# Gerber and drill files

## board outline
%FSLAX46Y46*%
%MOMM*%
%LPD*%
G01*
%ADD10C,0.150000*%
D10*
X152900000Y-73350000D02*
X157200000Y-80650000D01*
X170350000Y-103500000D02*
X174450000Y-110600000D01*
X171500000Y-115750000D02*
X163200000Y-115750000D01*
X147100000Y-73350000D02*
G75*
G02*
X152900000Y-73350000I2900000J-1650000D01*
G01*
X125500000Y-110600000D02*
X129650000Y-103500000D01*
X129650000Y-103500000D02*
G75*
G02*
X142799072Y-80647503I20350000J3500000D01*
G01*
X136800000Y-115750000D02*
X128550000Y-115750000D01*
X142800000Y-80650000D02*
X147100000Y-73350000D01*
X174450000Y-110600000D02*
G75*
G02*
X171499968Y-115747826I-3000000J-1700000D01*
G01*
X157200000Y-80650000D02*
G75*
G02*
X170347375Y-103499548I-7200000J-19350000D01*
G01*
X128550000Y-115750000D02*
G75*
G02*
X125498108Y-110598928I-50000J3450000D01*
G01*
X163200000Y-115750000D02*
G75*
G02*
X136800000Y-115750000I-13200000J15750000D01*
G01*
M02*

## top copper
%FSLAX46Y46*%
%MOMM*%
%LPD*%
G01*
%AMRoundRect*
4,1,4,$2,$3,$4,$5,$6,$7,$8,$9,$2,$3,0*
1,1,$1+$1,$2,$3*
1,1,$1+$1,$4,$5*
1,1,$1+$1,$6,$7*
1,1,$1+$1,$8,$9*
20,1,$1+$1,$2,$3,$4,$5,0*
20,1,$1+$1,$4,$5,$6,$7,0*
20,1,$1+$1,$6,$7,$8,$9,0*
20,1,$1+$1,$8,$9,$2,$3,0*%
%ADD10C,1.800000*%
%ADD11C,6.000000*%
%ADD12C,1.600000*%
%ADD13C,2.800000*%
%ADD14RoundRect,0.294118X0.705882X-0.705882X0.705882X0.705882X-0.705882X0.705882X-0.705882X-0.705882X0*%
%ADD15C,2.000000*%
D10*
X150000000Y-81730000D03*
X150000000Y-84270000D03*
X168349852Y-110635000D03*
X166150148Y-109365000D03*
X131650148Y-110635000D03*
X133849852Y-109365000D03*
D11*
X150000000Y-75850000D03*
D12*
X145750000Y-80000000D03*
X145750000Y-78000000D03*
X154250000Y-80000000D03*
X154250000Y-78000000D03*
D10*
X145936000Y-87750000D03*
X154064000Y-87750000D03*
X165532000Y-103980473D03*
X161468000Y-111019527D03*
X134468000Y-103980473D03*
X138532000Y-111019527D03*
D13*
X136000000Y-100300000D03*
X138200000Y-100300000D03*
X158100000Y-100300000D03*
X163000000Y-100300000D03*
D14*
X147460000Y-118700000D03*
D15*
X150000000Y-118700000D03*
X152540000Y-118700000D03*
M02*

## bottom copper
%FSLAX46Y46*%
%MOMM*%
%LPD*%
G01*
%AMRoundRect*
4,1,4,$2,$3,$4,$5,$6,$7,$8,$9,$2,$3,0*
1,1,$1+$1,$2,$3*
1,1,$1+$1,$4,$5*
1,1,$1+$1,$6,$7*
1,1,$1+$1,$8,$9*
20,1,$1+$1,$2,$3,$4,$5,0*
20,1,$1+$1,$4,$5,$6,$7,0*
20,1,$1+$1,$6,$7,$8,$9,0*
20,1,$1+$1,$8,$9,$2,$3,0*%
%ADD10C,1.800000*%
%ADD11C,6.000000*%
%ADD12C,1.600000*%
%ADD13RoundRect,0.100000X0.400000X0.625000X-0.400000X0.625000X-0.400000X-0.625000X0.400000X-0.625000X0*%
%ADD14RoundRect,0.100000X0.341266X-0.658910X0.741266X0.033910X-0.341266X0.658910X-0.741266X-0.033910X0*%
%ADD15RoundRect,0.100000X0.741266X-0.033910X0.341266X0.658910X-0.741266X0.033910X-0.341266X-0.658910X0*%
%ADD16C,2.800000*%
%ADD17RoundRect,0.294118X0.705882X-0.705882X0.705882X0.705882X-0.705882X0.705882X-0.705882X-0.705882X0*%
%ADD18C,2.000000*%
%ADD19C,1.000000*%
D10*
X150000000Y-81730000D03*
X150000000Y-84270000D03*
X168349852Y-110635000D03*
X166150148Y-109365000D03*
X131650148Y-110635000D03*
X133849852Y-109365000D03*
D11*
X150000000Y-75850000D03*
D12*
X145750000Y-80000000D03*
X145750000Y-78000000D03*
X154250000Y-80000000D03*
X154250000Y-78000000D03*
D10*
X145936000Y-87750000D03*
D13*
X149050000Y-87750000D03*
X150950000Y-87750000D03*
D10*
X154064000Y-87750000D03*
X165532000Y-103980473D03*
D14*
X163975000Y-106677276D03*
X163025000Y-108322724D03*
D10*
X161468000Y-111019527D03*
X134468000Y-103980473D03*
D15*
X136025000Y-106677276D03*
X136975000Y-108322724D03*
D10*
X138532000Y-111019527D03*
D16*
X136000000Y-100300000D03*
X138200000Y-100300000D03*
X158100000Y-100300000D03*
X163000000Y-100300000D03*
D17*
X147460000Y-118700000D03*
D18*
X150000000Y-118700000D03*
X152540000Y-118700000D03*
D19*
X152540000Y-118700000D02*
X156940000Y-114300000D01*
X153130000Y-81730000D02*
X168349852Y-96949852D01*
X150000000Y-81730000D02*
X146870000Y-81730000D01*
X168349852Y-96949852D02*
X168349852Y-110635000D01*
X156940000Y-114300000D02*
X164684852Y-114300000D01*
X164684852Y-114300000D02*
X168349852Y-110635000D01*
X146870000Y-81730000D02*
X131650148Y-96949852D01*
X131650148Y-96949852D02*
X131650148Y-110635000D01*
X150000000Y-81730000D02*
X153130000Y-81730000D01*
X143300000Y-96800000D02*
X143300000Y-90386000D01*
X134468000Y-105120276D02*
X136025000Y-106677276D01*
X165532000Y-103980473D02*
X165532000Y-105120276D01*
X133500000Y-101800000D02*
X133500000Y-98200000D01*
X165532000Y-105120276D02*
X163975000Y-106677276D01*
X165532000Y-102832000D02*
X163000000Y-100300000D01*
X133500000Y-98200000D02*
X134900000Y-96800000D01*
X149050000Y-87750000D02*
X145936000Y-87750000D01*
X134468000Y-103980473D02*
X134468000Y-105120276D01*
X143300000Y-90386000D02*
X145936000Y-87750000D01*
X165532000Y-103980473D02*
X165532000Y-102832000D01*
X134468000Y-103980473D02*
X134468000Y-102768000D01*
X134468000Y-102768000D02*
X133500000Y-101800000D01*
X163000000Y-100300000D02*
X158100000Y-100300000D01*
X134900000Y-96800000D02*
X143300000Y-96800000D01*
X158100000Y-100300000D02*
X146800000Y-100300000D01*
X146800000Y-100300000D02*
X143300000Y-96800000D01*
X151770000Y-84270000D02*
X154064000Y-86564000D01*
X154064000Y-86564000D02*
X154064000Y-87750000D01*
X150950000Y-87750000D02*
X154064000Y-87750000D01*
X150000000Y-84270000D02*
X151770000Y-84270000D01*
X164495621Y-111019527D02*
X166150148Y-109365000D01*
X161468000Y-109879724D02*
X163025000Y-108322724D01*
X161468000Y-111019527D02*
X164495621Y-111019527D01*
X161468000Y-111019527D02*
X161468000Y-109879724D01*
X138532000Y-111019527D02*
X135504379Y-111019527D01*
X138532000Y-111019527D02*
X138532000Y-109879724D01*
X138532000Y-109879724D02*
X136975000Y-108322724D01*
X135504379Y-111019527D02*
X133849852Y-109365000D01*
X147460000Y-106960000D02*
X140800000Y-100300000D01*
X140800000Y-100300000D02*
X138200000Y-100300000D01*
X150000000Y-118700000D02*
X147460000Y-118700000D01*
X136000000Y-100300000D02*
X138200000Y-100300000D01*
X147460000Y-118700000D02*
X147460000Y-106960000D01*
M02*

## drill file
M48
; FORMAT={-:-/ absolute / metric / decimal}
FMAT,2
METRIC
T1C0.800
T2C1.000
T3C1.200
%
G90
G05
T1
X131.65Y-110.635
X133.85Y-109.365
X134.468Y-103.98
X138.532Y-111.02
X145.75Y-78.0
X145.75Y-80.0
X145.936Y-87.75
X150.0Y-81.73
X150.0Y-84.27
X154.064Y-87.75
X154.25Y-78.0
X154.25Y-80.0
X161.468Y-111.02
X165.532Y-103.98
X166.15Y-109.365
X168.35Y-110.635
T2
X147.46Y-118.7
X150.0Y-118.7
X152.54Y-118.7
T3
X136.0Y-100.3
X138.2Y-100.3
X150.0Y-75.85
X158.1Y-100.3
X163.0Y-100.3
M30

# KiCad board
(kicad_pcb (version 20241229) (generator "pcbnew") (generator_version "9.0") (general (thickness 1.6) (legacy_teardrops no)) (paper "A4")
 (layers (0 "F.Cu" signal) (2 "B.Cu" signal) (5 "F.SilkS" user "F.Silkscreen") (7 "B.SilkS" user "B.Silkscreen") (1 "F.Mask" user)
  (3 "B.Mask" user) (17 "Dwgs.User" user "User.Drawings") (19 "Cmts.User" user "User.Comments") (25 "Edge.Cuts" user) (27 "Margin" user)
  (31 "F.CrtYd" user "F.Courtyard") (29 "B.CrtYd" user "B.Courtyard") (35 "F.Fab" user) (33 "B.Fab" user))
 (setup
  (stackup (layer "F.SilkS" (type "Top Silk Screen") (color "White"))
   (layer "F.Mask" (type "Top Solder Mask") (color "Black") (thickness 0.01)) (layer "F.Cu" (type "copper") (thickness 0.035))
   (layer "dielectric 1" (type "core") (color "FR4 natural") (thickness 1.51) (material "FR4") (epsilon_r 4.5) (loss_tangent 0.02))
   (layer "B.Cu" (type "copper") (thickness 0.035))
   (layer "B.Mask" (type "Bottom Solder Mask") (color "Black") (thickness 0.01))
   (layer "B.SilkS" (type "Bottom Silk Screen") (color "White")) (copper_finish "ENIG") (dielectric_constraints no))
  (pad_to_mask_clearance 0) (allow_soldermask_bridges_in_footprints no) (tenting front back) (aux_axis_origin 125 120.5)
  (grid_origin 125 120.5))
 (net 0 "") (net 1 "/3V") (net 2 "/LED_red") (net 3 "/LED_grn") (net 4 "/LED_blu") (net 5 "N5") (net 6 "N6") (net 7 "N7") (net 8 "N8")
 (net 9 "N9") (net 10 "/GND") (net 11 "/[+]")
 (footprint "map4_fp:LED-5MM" (layer "F.Cu") (at 150 83 -90)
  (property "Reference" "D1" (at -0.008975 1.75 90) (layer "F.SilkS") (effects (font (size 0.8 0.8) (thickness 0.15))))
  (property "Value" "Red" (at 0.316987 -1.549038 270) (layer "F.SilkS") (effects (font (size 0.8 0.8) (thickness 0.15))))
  (pad "1" thru_hole circle (at -1.27 0 270) (size 1.8 1.8) (drill 0.8) (layers "*.Cu" "*.Mask") (remove_unused_layers no) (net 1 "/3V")
   (solder_mask_margin 0.1) (clearance 0.1))
  (pad "2" thru_hole circle (at 1.27 0 270) (size 1.8 1.8) (drill 0.8) (layers "*.Cu" "*.Mask") (remove_unused_layers no) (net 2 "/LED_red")
   (solder_mask_margin 0.1) (clearance 0.1)))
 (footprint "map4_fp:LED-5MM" (layer "F.Cu") (at 167.25 110 150)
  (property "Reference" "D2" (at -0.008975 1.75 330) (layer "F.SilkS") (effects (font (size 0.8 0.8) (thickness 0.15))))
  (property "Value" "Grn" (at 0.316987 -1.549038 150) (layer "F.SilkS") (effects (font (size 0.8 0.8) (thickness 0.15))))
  (pad "1" thru_hole circle (at -1.27 0 150) (size 1.8 1.8) (drill 0.8) (layers "*.Cu" "*.Mask") (remove_unused_layers no) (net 1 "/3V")
   (solder_mask_margin 0.1) (clearance 0.1))
  (pad "2" thru_hole circle (at 1.27 0 150) (size 1.8 1.8) (drill 0.8) (layers "*.Cu" "*.Mask") (remove_unused_layers no) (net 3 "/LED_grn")
   (solder_mask_margin 0.1) (clearance 0.1)))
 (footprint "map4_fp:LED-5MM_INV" (layer "F.Cu") (at 132.75 110 30)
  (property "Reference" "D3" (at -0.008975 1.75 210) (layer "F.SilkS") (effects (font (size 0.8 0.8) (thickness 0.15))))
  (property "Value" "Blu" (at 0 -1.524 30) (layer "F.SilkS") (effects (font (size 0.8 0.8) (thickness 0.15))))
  (pad "1" thru_hole circle (at -1.27 0 30) (size 1.8 1.8) (drill 0.8) (layers "*.Cu" "*.Mask") (remove_unused_layers no) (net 1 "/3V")
   (solder_mask_margin 0.1) (clearance 0.1))
  (pad "2" thru_hole circle (at 1.27 0 30) (size 1.8 1.8) (drill 0.8) (layers "*.Cu" "*.Mask") (remove_unused_layers no) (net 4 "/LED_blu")
   (solder_mask_margin 0.1) (clearance 0.1)))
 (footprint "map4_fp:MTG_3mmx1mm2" (layer "F.Cu") (at 150 75.85)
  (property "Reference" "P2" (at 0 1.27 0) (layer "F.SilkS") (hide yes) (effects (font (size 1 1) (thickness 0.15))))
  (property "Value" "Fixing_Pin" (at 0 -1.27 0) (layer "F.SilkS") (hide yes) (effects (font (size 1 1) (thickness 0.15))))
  (pad "1" thru_hole circle (at 0 0) (size 6 6) (drill 1.2) (layers "*.Cu" "*.Mask") (remove_unused_layers no) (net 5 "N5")))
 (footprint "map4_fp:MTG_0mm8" (layer "F.Cu") (at 145.75 80)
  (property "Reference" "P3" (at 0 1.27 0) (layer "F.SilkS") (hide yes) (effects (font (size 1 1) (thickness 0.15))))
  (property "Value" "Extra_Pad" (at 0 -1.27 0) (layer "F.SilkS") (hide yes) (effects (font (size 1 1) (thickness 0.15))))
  (pad "1" thru_hole circle (at 0 0) (size 1.6 1.6) (drill 0.8) (layers "*.Cu" "*.Mask") (remove_unused_layers no) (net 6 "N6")))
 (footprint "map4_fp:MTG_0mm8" (layer "F.Cu") (at 145.75 78)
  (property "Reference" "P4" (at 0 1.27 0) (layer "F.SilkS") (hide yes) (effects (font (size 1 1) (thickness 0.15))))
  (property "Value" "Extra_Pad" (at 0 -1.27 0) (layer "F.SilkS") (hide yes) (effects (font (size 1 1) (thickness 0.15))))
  (pad "1" thru_hole circle (at 0 0) (size 1.6 1.6) (drill 0.8) (layers "*.Cu" "*.Mask") (remove_unused_layers no) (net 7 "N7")))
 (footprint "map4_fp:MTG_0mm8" (layer "F.Cu") (at 154.25 80)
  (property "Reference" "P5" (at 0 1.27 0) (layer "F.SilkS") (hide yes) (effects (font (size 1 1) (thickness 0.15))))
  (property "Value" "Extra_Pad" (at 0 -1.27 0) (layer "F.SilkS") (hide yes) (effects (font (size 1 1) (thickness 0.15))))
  (pad "1" thru_hole circle (at 0 0) (size 1.6 1.6) (drill 0.8) (layers "*.Cu" "*.Mask") (remove_unused_layers no) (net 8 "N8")))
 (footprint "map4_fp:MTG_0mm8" (layer "F.Cu") (at 154.25 78)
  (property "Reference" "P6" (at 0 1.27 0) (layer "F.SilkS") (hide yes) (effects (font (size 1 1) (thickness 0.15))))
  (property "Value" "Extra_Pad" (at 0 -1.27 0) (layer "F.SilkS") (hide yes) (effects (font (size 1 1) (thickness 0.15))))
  (pad "1" thru_hole circle (at 0 0) (size 1.6 1.6) (drill 0.8) (layers "*.Cu" "*.Mask") (remove_unused_layers no) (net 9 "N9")))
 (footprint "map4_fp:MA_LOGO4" (layer "F.Cu") (at 150 97.5)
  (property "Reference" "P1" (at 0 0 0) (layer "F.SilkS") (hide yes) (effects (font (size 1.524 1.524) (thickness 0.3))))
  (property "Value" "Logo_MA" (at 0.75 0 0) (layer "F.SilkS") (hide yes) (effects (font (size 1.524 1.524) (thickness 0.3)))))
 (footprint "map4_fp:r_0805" (layer "B.Cu") (at 150 87.75)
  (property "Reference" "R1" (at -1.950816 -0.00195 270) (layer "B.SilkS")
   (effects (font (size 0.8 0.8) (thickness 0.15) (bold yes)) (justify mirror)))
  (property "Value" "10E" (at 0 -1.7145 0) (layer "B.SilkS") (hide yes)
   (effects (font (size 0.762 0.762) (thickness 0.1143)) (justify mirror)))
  (pad "1" thru_hole circle (at -4.064 0 180) (size 1.8 1.8) (drill 0.8) (layers "*.Cu" "*.Mask") (remove_unused_layers no) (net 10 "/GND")
   (solder_mask_margin 0.1) (clearance 0.1))
  (pad "1" smd roundrect (at -0.95 0 180) (size 1 1.45) (layers "B.Cu" "B.Mask" "B.Paste") (roundrect_rratio 0.1) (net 10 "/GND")
   (solder_mask_margin 0.05) (clearance 0.05))
  (pad "2" smd roundrect (at 0.95 0 180) (size 1 1.45) (layers "B.Cu" "B.Mask" "B.Paste") (roundrect_rratio 0.1) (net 2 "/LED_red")
   (solder_mask_margin 0.05) (clearance 0.05))
  (pad "2" thru_hole circle (at 4.064 0 180) (size 1.8 1.8) (drill 0.8) (layers "*.Cu" "*.Mask") (remove_unused_layers no)
   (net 2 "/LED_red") (solder_mask_margin 0.1) (clearance 0.1)))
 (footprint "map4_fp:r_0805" (layer "B.Cu") (at 163.5 107.5 -120)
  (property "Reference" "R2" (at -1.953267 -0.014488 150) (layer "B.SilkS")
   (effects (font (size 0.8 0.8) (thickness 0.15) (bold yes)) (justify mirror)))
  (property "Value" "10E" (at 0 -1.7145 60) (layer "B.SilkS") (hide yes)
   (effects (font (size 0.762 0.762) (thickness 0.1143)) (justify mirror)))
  (pad "1" thru_hole circle (at -4.064 0 60) (size 1.8 1.8) (drill 0.8) (layers "*.Cu" "*.Mask") (remove_unused_layers no) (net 10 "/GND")
   (solder_mask_margin 0.1) (clearance 0.1))
  (pad "1" smd roundrect (at -0.95 0 60) (size 1 1.45) (layers "B.Cu" "B.Mask" "B.Paste") (roundrect_rratio 0.1) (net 10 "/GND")
   (solder_mask_margin 0.05) (clearance 0.05))
  (pad "2" smd roundrect (at 0.95 0 60) (size 1 1.45) (layers "B.Cu" "B.Mask" "B.Paste") (roundrect_rratio 0.1) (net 3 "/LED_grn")
   (solder_mask_margin 0.05) (clearance 0.05))
  (pad "2" thru_hole circle (at 4.064 0 60) (size 1.8 1.8) (drill 0.8) (layers "*.Cu" "*.Mask") (remove_unused_layers no) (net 3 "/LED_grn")
   (solder_mask_margin 0.1) (clearance 0.1)))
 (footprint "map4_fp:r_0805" (layer "B.Cu") (at 136.5 107.5 -60)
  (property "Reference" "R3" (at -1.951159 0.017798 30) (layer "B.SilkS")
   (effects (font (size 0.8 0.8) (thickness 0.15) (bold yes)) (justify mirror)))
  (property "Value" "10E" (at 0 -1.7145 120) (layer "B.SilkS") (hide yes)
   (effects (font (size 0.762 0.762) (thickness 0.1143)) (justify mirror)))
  (pad "1" thru_hole circle (at -4.064 0 120) (size 1.8 1.8) (drill 0.8) (layers "*.Cu" "*.Mask") (remove_unused_layers no) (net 10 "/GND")
   (solder_mask_margin 0.1) (clearance 0.1))
  (pad "1" smd roundrect (at -0.95 0 120) (size 1 1.45) (layers "B.Cu" "B.Mask" "B.Paste") (roundrect_rratio 0.1) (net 10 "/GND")
   (solder_mask_margin 0.05) (clearance 0.05))
  (pad "2" smd roundrect (at 0.95 0 120) (size 1 1.45) (layers "B.Cu" "B.Mask" "B.Paste") (roundrect_rratio 0.1) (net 4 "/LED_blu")
   (solder_mask_margin 0.05) (clearance 0.05))
  (pad "2" thru_hole circle (at 4.064 0 120) (size 1.8 1.8) (drill 0.8) (layers "*.Cu" "*.Mask") (remove_unused_layers no)
   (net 4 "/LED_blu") (solder_mask_margin 0.1) (clearance 0.1)))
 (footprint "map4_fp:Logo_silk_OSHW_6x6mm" (layer "B.Cu") (at 150 114 180)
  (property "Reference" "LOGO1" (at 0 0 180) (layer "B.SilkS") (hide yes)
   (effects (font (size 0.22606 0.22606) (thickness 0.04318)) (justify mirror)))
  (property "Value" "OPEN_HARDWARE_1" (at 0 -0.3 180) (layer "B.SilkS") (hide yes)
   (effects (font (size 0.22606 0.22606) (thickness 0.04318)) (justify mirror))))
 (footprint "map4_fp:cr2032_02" (layer "B.Cu") (at 150 100.3 90)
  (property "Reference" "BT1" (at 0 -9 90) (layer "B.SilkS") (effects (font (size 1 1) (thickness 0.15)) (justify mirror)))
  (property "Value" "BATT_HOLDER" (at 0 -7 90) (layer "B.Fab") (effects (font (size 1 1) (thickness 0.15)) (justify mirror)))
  (pad "1" thru_hole circle (at 0 -14 270) (size 2.8 2.8) (drill 1.2) (layers "*.Cu" "*.Mask") (remove_unused_layers no) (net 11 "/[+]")
   (solder_mask_margin 0.1) (clearance 0.1))
  (pad "1" thru_hole circle (at 0 -11.8 270) (size 2.8 2.8) (drill 1.2) (layers "*.Cu" "*.Mask") (remove_unused_layers no) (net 11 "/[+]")
   (solder_mask_margin 0.1) (clearance 0.1))
  (pad "2" thru_hole circle (at 0 8.1 270) (size 2.8 2.8) (drill 1.2) (layers "*.Cu" "*.Mask") (remove_unused_layers no) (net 10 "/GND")
   (solder_mask_margin 0.1) (clearance 0.1))
  (pad "2" thru_hole circle (at 0 13 270) (size 2.8 2.8) (drill 1.2) (layers "*.Cu" "*.Mask") (remove_unused_layers no) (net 10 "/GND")
   (solder_mask_margin 0.1) (clearance 0.1)))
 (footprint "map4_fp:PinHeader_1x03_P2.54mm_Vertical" (layer "B.Cu") (at 147.46 118.7 -90)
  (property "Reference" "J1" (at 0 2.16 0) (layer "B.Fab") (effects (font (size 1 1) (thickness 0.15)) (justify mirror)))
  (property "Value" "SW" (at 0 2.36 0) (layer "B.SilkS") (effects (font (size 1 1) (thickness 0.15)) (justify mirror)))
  (pad "1" thru_hole roundrect (at 0 0 90) (size 2 2) (drill 1) (layers "*.Cu" "*.Mask") (remove_unused_layers no)
   (roundrect_rratio 0.1470588235) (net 11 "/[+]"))
  (pad "2" thru_hole circle (at 0 -2.54 90) (size 2 2) (drill 1) (layers "*.Cu" "*.Mask") (remove_unused_layers no) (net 11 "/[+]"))
  (pad "3" thru_hole circle (at 0 -5.08 90) (size 2 2) (drill 1) (layers "*.Cu" "*.Mask") (remove_unused_layers no) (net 1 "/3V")))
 (gr_line (start 152.9 73.35) (end 157.2 80.65) (stroke (width 0.15) (type solid)) (layer "Edge.Cuts"))
 (gr_line (start 170.35 103.5) (end 174.45 110.6) (stroke (width 0.15) (type solid)) (layer "Edge.Cuts"))
 (gr_line (start 171.5 115.75) (end 163.2 115.75) (stroke (width 0.15) (type solid)) (layer "Edge.Cuts"))
 (gr_arc (start 147.1 73.35) (mid 150 71.66346) (end 152.9 73.35) (stroke (width 0.15) (type solid)) (layer "Edge.Cuts"))
 (gr_line (start 125.5 110.6) (end 129.65 103.5) (stroke (width 0.15) (type solid)) (layer "Edge.Cuts"))
 (gr_arc (start 129.65 103.5) (mid 132.102443 89.701945) (end 142.799072 80.647503) (stroke (width 0.15) (type solid)) (layer "Edge.Cuts"))
 (gr_line (start 136.8 115.75) (end 128.55 115.75) (stroke (width 0.15) (type solid)) (layer "Edge.Cuts"))
 (gr_line (start 142.8 80.65) (end 147.1 73.35) (stroke (width 0.15) (type solid)) (layer "Edge.Cuts"))
 (gr_arc (start 174.45 110.6) (mid 174.441756 114.014467) (end 171.499968 115.747826) (stroke (width 0.15) (type solid)) (layer "Edge.Cuts"))
 (gr_arc (start 157.2 80.65) (mid 167.895249 89.703274) (end 170.347375 103.499548) (stroke (width 0.15) (type solid)) (layer "Edge.Cuts"))
 (gr_arc (start 128.55 115.75) (mid 125.531532 114.058749) (end 125.498108 110.598928) (stroke (width 0.15) (type solid))
  (layer "Edge.Cuts"))
 (gr_arc (start 163.2 115.75) (mid 150 120.55) (end 136.8 115.75) (stroke (width 0.15) (type solid)) (layer "Edge.Cuts"))
 (segment (start 152.54 118.7) (end 156.94 114.3) (width 1) (layer "B.Cu") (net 1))
 (segment (start 153.13 81.73) (end 168.349852 96.949852) (width 1) (layer "B.Cu") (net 1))
 (segment (start 150 81.73) (end 146.87 81.73) (width 1) (layer "B.Cu") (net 1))
 (segment (start 168.349852 96.949852) (end 168.349852 110.635) (width 1) (layer "B.Cu") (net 1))
 (segment (start 156.94 114.3) (end 164.684852 114.3) (width 1) (layer "B.Cu") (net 1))
 (segment (start 164.684852 114.3) (end 168.349852 110.635) (width 1) (layer "B.Cu") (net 1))
 (segment (start 146.87 81.73) (end 131.650148 96.949852) (width 1) (layer "B.Cu") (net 1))
 (segment (start 131.650148 96.949852) (end 131.650148 110.635) (width 1) (layer "B.Cu") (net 1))
 (segment (start 150 81.73) (end 153.13 81.73) (width 1) (layer "B.Cu") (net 1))
 (segment (start 143.3 96.8) (end 143.3 90.386) (width 1) (layer "B.Cu") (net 10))
 (segment (start 134.468 105.120276) (end 136.025 106.677276) (width 1) (layer "B.Cu") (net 10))
 (segment (start 165.532 103.980473) (end 165.532 105.120276) (width 1) (layer "B.Cu") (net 10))
 (segment (start 133.5 101.8) (end 133.5 98.2) (width 1) (layer "B.Cu") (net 10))
 (segment (start 165.532 105.120276) (end 163.975 106.677276) (width 1) (layer "B.Cu") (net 10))
 (segment (start 165.532 102.832) (end 163 100.3) (width 1) (layer "B.Cu") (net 10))
 (segment (start 133.5 98.2) (end 134.9 96.8) (width 1) (layer "B.Cu") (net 10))
 (segment (start 149.05 87.75) (end 145.936 87.75) (width 1) (layer "B.Cu") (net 10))
 (segment (start 134.468 103.980473) (end 134.468 105.120276) (width 1) (layer "B.Cu") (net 10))
 (segment (start 143.3 90.386) (end 145.936 87.75) (width 1) (layer "B.Cu") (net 10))
 (segment (start 165.532 103.980473) (end 165.532 102.832) (width 1) (layer "B.Cu") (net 10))
 (segment (start 134.468 103.980473) (end 134.468 102.768) (width 1) (layer "B.Cu") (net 10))
 (segment (start 134.468 102.768) (end 133.5 101.8) (width 1) (layer "B.Cu") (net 10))
 (segment (start 163 100.3) (end 158.1 100.3) (width 1) (layer "B.Cu") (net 10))
 (segment (start 134.9 96.8) (end 143.3 96.8) (width 1) (layer "B.Cu") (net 10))
 (segment (start 158.1 100.3) (end 146.8 100.3) (width 1) (layer "B.Cu") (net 10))
 (segment (start 146.8 100.3) (end 143.3 96.8) (width 1) (layer "B.Cu") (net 10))
 (segment (start 151.77 84.27) (end 154.064 86.564) (width 1) (layer "B.Cu") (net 2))
 (segment (start 154.064 86.564) (end 154.064 87.75) (width 1) (layer "B.Cu") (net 2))
 (segment (start 150.95 87.75) (end 154.064 87.75) (width 1) (layer "B.Cu") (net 2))
 (segment (start 150 84.27) (end 151.77 84.27) (width 1) (layer "B.Cu") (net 2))
 (segment (start 164.495621 111.019527) (end 166.150148 109.365) (width 1) (layer "B.Cu") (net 3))
 (segment (start 161.468 109.879724) (end 163.025 108.322724) (width 1) (layer "B.Cu") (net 3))
 (segment (start 161.468 111.019527) (end 164.495621 111.019527) (width 1) (layer "B.Cu") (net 3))
 (segment (start 161.468 111.019527) (end 161.468 109.879724) (width 1) (layer "B.Cu") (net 3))
 (segment (start 138.532 111.019527) (end 135.504379 111.019527) (width 1) (layer "B.Cu") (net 4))
 (segment (start 138.532 111.019527) (end 138.532 109.879724) (width 1) (layer "B.Cu") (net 4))
 (segment (start 138.532 109.879724) (end 136.975 108.322724) (width 1) (layer "B.Cu") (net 4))
 (segment (start 135.504379 111.019527) (end 133.849852 109.365) (width 1) (layer "B.Cu") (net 4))
 (segment (start 147.46 106.96) (end 140.8 100.3) (width 1) (layer "B.Cu") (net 11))
 (segment (start 140.8 100.3) (end 138.2 100.3) (width 1) (layer "B.Cu") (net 11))
 (segment (start 150 118.7) (end 147.46 118.7) (width 1) (layer "B.Cu") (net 11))
 (segment (start 136 100.3) (end 138.2 100.3) (width 1) (layer "B.Cu") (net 11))
 (segment (start 147.46 118.7) (end 147.46 106.96) (width 1) (layer "B.Cu") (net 11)))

